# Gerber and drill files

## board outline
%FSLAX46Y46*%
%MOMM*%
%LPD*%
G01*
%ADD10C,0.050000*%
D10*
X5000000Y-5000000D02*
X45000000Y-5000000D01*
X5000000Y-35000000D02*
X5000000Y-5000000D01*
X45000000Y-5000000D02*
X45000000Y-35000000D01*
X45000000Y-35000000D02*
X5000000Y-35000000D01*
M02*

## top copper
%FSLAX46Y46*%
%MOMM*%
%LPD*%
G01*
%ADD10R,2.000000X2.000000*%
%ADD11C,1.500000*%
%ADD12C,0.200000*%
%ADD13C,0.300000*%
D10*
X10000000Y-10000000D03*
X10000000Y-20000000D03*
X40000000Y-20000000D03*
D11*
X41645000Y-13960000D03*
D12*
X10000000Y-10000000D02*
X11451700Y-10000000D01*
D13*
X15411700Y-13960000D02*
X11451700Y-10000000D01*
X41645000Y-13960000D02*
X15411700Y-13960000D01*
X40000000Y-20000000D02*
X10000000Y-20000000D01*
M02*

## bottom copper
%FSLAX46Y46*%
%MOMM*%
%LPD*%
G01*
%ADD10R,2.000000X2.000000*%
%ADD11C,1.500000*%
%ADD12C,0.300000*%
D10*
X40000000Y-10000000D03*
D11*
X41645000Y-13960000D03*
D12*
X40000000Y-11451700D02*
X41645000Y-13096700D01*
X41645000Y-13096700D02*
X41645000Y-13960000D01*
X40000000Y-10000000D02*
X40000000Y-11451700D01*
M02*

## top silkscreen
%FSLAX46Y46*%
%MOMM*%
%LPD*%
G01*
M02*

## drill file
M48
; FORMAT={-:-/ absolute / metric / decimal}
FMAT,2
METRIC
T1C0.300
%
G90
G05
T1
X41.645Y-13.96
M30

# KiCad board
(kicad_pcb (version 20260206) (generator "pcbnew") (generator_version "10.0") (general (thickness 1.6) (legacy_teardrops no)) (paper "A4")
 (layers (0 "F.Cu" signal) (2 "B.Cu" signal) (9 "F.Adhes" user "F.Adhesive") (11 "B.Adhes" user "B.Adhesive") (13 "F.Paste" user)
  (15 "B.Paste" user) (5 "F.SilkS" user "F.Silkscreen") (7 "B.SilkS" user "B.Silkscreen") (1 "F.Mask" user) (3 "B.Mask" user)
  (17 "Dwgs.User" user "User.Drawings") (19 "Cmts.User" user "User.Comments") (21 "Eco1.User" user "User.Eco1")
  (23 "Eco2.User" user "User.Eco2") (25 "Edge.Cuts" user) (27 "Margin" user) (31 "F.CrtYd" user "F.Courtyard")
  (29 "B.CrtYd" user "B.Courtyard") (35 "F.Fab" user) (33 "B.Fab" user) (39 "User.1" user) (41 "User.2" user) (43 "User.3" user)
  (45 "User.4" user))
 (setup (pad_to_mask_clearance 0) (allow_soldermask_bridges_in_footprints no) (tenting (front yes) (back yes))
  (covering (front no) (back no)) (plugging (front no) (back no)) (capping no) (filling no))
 (gr_line (start 5 5) (end 45 5) (stroke (width 0.05) (type default)) (layer "Edge.Cuts"))
 (gr_line (start 5 35) (end 5 5) (stroke (width 0.05) (type default)) (layer "Edge.Cuts"))
 (gr_line (start 45 5) (end 45 35) (stroke (width 0.05) (type default)) (layer "Edge.Cuts"))
 (gr_line (start 45 35) (end 5 35) (stroke (width 0.05) (type default)) (layer "Edge.Cuts"))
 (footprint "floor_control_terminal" (layer "F.Cu") (at 10 10)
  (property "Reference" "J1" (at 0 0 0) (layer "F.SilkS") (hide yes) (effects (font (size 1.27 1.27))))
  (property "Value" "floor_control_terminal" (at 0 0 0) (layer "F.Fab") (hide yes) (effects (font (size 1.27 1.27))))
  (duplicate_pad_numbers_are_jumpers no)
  (pad "1" smd rect (at 0 0) (size 2 2) (layers "F.Cu" "F.Paste" "F.Mask") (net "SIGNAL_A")))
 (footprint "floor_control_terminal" (layer "B.Cu") (at 40 10)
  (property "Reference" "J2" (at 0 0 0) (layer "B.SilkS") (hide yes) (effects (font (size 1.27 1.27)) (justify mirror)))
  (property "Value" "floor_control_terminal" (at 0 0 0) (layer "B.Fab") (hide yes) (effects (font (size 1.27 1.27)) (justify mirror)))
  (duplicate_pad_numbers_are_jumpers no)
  (pad "1" smd rect (at 0 0) (size 2 2) (layers "B.Cu" "B.Paste" "B.Mask") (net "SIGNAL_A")))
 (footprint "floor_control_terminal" (layer "F.Cu") (at 10 20)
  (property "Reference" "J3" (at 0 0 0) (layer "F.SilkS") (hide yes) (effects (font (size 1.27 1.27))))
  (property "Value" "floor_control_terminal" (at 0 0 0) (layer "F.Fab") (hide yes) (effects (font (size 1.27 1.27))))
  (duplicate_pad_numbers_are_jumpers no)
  (pad "1" smd rect (at 0 0) (size 2 2) (layers "F.Cu" "F.Paste" "F.Mask") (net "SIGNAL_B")))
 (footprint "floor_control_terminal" (layer "F.Cu") (at 40 20)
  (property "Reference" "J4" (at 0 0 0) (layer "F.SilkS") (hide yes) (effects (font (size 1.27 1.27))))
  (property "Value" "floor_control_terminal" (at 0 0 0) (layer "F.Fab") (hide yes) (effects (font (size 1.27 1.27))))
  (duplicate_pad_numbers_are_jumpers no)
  (pad "1" smd rect (at 0 0) (size 2 2) (layers "F.Cu" "F.Paste" "F.Mask") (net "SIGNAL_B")))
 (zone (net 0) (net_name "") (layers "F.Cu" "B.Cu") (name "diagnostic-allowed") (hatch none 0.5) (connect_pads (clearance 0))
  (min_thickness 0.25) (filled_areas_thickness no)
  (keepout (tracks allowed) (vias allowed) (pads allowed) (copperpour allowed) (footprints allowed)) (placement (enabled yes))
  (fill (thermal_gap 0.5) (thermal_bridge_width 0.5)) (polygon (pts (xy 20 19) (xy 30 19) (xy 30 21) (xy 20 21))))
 (segment (start 10 10) (end 11.4517 10) (width 0.2) (layer "F.Cu") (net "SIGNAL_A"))
 (segment (start 15.4117 13.96) (end 11.4517 10) (width 0.3) (layer "F.Cu") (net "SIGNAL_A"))
 (segment (start 41.645 13.96) (end 15.4117 13.96) (width 0.3) (layer "F.Cu") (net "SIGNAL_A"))
 (via (at 41.645 13.96) (size 1.5) (drill 0.3) (layers "F.Cu" "B.Cu") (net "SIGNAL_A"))
 (segment (start 40 11.4517) (end 41.645 13.0967) (width 0.3) (layer "B.Cu") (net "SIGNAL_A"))
 (segment (start 41.645 13.0967) (end 41.645 13.96) (width 0.3) (layer "B.Cu") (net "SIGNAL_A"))
 (segment (start 40 10) (end 40 11.4517) (width 0.3) (layer "B.Cu") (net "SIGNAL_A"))
 (segment (start 40 20) (end 10 20) (width 0.3) (layer "F.Cu") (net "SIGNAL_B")))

